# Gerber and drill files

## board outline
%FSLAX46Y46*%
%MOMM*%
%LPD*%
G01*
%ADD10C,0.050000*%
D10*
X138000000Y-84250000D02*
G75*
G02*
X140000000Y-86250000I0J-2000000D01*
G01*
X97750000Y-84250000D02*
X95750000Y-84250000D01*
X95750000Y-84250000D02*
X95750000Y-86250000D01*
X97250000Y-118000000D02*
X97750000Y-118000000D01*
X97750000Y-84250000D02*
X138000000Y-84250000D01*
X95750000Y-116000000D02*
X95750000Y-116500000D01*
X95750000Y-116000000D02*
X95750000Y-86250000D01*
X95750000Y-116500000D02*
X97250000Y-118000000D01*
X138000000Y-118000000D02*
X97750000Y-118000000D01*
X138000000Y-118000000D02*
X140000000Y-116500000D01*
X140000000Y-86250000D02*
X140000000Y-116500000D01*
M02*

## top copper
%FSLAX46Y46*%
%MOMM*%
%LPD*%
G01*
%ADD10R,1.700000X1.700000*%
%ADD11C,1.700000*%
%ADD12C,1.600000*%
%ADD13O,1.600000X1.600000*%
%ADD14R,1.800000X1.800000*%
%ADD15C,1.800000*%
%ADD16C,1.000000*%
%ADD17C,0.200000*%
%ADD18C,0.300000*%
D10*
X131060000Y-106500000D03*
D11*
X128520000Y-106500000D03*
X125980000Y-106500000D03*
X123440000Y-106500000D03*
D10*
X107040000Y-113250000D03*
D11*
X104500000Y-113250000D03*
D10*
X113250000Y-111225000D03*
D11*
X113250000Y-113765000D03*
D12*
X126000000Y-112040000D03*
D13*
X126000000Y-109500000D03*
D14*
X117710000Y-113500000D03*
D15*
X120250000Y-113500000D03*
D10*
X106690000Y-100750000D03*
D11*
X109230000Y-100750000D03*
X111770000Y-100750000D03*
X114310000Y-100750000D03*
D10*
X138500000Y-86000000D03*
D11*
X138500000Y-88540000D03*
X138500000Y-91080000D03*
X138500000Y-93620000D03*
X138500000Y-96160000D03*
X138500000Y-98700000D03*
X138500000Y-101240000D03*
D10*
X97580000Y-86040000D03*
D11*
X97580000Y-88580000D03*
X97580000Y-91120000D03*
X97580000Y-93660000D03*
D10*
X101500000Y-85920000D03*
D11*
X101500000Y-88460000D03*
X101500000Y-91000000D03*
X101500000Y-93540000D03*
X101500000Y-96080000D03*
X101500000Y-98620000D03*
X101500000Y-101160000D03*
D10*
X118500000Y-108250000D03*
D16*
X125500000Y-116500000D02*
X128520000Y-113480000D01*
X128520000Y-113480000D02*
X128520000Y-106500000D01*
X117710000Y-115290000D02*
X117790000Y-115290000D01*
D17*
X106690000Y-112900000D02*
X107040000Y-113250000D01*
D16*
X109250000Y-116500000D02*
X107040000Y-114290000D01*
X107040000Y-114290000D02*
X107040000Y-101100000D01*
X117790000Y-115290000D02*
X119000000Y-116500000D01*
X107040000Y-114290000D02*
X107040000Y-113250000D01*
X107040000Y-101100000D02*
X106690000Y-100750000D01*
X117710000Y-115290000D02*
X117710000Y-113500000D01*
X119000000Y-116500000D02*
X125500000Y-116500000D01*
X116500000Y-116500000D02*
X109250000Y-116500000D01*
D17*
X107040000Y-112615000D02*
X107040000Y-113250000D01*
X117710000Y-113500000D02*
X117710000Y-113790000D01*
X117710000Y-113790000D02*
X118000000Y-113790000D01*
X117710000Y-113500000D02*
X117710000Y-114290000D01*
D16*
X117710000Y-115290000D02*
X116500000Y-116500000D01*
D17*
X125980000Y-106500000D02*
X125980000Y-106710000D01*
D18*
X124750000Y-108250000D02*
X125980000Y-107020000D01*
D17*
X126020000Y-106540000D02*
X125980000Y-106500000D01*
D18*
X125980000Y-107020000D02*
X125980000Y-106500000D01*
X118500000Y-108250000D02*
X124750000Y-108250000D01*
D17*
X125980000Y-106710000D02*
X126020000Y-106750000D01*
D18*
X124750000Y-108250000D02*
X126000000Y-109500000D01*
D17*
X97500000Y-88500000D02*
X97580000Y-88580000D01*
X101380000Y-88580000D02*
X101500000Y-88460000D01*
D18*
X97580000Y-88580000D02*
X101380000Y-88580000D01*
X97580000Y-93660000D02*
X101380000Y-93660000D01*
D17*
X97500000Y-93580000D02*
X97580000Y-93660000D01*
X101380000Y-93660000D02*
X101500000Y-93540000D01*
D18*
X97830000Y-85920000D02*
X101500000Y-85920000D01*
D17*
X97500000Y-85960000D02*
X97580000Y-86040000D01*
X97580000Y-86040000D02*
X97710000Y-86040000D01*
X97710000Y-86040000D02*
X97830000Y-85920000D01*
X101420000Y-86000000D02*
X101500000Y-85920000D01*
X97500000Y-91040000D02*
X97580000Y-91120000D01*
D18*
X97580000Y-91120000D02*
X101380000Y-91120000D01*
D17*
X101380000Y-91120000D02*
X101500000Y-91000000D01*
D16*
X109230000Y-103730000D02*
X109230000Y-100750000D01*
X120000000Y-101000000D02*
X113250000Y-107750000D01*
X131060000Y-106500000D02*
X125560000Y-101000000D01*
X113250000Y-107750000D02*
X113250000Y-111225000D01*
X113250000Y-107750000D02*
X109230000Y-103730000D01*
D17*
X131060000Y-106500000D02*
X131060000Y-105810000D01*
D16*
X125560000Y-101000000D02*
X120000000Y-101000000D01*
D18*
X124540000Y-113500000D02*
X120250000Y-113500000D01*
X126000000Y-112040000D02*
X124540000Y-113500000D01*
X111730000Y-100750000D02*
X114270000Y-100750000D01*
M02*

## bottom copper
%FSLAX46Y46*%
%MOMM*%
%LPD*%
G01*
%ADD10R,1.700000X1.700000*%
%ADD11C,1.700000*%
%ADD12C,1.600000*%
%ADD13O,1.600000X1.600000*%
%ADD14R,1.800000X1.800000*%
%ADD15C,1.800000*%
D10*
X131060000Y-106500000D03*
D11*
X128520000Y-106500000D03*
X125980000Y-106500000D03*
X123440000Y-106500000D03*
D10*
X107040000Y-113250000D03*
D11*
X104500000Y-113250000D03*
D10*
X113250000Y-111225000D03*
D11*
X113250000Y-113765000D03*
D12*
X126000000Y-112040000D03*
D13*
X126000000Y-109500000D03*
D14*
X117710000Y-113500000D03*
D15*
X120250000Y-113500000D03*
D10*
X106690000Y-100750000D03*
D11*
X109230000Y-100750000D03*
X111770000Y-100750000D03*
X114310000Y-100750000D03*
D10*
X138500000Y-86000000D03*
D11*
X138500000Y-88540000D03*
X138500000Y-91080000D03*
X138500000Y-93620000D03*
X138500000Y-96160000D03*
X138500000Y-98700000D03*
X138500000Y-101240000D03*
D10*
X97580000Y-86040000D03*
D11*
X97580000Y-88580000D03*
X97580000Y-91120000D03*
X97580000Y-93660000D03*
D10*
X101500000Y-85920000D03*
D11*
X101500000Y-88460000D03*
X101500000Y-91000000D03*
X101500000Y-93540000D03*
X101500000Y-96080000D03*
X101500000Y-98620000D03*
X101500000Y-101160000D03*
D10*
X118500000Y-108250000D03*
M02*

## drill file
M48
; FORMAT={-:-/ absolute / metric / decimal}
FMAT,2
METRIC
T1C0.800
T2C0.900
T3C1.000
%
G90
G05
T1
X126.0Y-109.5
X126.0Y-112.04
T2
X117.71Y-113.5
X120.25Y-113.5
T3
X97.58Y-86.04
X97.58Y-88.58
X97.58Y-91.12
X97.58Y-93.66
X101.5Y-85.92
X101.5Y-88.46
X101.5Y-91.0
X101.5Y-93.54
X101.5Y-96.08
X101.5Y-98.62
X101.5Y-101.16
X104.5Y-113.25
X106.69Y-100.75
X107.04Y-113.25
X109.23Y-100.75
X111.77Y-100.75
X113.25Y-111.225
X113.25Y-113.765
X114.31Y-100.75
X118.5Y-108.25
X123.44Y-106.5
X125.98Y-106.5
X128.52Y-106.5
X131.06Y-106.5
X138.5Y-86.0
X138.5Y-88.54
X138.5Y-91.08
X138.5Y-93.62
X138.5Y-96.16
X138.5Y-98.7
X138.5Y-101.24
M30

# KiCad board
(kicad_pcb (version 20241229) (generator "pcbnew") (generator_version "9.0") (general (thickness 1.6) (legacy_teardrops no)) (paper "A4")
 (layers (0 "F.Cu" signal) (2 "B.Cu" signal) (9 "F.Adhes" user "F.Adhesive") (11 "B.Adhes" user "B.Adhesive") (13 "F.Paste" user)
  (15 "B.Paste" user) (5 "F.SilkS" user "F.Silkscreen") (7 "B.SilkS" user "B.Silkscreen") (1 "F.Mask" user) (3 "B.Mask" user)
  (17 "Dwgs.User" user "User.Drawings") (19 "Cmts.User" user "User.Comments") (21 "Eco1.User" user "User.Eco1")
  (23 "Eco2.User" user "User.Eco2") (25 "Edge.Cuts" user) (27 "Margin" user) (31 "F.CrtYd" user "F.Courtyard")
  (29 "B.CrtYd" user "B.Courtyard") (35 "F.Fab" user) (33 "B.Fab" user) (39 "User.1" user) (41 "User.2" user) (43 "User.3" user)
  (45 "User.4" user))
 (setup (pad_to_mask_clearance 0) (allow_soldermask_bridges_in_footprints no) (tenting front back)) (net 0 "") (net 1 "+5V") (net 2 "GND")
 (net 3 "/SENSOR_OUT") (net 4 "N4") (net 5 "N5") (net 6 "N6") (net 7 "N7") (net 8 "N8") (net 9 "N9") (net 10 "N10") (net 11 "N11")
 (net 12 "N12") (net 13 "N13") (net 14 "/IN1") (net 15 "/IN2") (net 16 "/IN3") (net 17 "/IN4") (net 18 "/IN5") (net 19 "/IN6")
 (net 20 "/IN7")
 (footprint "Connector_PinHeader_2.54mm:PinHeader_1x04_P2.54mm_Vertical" (layer "F.Cu") (at 131.06 106.5 -90)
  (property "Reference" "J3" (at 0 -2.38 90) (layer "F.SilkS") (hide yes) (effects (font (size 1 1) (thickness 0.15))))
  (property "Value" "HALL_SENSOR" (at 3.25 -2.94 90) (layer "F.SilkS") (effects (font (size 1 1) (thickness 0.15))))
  (pad "1" thru_hole rect (at 0 0 270) (size 1.7 1.7) (drill 1) (layers "*.Cu" "*.Mask") (remove_unused_layers no) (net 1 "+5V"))
  (pad "2" thru_hole circle (at 0 2.54 270) (size 1.7 1.7) (drill 1) (layers "*.Cu" "*.Mask") (remove_unused_layers no) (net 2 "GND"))
  (pad "3" thru_hole circle (at 0 5.08 270) (size 1.7 1.7) (drill 1) (layers "*.Cu" "*.Mask") (remove_unused_layers no)
   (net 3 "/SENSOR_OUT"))
  (pad "4" thru_hole circle (at 0 7.62 270) (size 1.7 1.7) (drill 1) (layers "*.Cu" "*.Mask") (remove_unused_layers no) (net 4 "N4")))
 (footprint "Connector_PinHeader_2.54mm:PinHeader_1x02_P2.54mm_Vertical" (layer "F.Cu") (at 107.04 113.25 -90)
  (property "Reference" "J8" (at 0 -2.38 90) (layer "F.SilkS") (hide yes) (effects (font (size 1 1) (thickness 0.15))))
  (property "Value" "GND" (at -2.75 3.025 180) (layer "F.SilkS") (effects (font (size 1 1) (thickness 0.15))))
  (pad "1" thru_hole rect (at 0 0 270) (size 1.7 1.7) (drill 1) (layers "*.Cu" "*.Mask") (remove_unused_layers no) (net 2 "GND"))
  (pad "2" thru_hole circle (at 0 2.54 270) (size 1.7 1.7) (drill 1) (layers "*.Cu" "*.Mask") (remove_unused_layers no)))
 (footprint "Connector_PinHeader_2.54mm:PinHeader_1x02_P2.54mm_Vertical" (layer "F.Cu") (at 113.25 111.225)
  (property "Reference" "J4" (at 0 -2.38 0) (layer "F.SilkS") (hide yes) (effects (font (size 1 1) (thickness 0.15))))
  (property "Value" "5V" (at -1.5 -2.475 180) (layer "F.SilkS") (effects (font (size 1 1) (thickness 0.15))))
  (pad "1" thru_hole rect (at 0 0) (size 1.7 1.7) (drill 1) (layers "*.Cu" "*.Mask") (remove_unused_layers no) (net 1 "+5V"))
  (pad "2" thru_hole circle (at 0 2.54) (size 1.7 1.7) (drill 1) (layers "*.Cu" "*.Mask") (remove_unused_layers no)))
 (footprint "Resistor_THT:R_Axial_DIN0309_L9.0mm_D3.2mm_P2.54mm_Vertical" (layer "F.Cu") (at 126 112.04 90)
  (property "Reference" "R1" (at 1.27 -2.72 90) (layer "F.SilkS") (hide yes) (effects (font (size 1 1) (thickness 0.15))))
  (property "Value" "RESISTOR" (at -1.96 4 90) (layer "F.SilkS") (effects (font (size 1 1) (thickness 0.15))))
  (pad "1" thru_hole circle (at 0 0 90) (size 1.6 1.6) (drill 0.8) (layers "*.Cu" "*.Mask") (remove_unused_layers no) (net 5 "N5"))
  (pad "2" thru_hole oval (at 2.54 0 90) (size 1.6 1.6) (drill 0.8) (layers "*.Cu" "*.Mask") (remove_unused_layers no) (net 3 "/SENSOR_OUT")))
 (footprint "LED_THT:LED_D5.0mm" (layer "F.Cu") (at 117.71 113.5)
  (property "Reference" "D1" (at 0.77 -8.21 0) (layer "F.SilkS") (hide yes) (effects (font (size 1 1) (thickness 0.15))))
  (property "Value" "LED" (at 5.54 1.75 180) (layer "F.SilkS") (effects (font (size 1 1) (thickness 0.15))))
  (pad "1" thru_hole rect (at 0 0) (size 1.8 1.8) (drill 0.9) (layers "*.Cu" "*.Mask") (remove_unused_layers no) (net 2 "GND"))
  (pad "2" thru_hole circle (at 2.54 0) (size 1.8 1.8) (drill 0.9) (layers "*.Cu" "*.Mask") (remove_unused_layers no) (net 5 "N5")))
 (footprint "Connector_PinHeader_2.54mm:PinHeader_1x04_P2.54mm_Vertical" (layer "F.Cu") (at 106.69 100.75 90)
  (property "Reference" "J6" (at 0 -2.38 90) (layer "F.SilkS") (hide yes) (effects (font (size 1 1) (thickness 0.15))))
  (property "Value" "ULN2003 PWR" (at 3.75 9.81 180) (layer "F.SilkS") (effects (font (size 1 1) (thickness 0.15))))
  (pad "1" thru_hole rect (at 0 0 90) (size 1.7 1.7) (drill 1) (layers "*.Cu" "*.Mask") (remove_unused_layers no) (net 2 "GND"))
  (pad "2" thru_hole circle (at 0 2.54 90) (size 1.7 1.7) (drill 1) (layers "*.Cu" "*.Mask") (remove_unused_layers no) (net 1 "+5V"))
  (pad "3" thru_hole circle (at 0 5.08 90) (size 1.7 1.7) (drill 1) (layers "*.Cu" "*.Mask") (remove_unused_layers no) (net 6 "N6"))
  (pad "4" thru_hole circle (at 0 7.62 90) (size 1.7 1.7) (drill 1) (layers "*.Cu" "*.Mask") (remove_unused_layers no) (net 6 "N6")))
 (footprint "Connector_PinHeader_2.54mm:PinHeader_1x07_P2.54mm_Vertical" (layer "F.Cu") (at 138.5 86)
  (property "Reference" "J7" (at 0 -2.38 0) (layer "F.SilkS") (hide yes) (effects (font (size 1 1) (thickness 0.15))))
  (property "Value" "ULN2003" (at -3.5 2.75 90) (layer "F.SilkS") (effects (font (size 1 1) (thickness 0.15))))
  (pad "1" thru_hole rect (at 0 0) (size 1.7 1.7) (drill 1) (layers "*.Cu" "*.Mask") (remove_unused_layers no) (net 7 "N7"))
  (pad "2" thru_hole circle (at 0 2.54) (size 1.7 1.7) (drill 1) (layers "*.Cu" "*.Mask") (remove_unused_layers no) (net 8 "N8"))
  (pad "3" thru_hole circle (at 0 5.08) (size 1.7 1.7) (drill 1) (layers "*.Cu" "*.Mask") (remove_unused_layers no) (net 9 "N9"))
  (pad "4" thru_hole circle (at 0 7.62) (size 1.7 1.7) (drill 1) (layers "*.Cu" "*.Mask") (remove_unused_layers no) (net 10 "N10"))
  (pad "5" thru_hole circle (at 0 10.16) (size 1.7 1.7) (drill 1) (layers "*.Cu" "*.Mask") (remove_unused_layers no) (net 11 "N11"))
  (pad "6" thru_hole circle (at 0 12.7) (size 1.7 1.7) (drill 1) (layers "*.Cu" "*.Mask") (remove_unused_layers no) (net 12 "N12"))
  (pad "7" thru_hole circle (at 0 15.24) (size 1.7 1.7) (drill 1) (layers "*.Cu" "*.Mask") (remove_unused_layers no) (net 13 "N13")))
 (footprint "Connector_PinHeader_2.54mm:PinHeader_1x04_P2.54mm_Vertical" (layer "F.Cu") (at 97.58 86.04)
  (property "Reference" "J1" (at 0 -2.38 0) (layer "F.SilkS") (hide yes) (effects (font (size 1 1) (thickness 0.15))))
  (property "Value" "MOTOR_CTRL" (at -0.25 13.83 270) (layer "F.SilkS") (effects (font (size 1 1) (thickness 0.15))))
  (pad "1" thru_hole rect (at 0 0) (size 1.7 1.7) (drill 1) (layers "*.Cu" "*.Mask") (remove_unused_layers no) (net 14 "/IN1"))
  (pad "2" thru_hole circle (at 0 2.54) (size 1.7 1.7) (drill 1) (layers "*.Cu" "*.Mask") (remove_unused_layers no) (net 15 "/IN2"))
  (pad "3" thru_hole circle (at 0 5.08) (size 1.7 1.7) (drill 1) (layers "*.Cu" "*.Mask") (remove_unused_layers no) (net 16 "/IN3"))
  (pad "4" thru_hole circle (at 0 7.62) (size 1.7 1.7) (drill 1) (layers "*.Cu" "*.Mask") (remove_unused_layers no) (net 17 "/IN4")))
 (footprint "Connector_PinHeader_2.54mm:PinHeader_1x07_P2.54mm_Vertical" (layer "F.Cu") (at 101.5 85.92)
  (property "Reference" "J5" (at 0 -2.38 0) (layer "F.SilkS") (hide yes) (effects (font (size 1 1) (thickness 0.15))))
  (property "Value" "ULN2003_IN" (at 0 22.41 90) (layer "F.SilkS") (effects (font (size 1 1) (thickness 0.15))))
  (pad "1" thru_hole rect (at 0 0) (size 1.7 1.7) (drill 1) (layers "*.Cu" "*.Mask") (remove_unused_layers no) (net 14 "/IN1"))
  (pad "2" thru_hole circle (at 0 2.54) (size 1.7 1.7) (drill 1) (layers "*.Cu" "*.Mask") (remove_unused_layers no) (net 15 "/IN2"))
  (pad "3" thru_hole circle (at 0 5.08) (size 1.7 1.7) (drill 1) (layers "*.Cu" "*.Mask") (remove_unused_layers no) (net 16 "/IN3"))
  (pad "4" thru_hole circle (at 0 7.62) (size 1.7 1.7) (drill 1) (layers "*.Cu" "*.Mask") (remove_unused_layers no) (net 17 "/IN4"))
  (pad "5" thru_hole circle (at 0 10.16) (size 1.7 1.7) (drill 1) (layers "*.Cu" "*.Mask") (remove_unused_layers no) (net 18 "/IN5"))
  (pad "6" thru_hole circle (at 0 12.7) (size 1.7 1.7) (drill 1) (layers "*.Cu" "*.Mask") (remove_unused_layers no) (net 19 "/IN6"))
  (pad "7" thru_hole circle (at 0 15.24) (size 1.7 1.7) (drill 1) (layers "*.Cu" "*.Mask") (remove_unused_layers no) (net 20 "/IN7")))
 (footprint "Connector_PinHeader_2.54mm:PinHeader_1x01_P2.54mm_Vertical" (layer "F.Cu") (at 118.5 108.25)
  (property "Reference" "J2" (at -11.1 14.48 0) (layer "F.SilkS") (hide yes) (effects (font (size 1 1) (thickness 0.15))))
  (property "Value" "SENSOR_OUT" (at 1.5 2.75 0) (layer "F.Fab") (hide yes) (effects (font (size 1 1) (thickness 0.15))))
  (pad "1" thru_hole rect (at 0 0) (size 1.7 1.7) (drill 1) (layers "*.Cu" "*.Mask") (remove_unused_layers no) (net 3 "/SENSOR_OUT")))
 (gr_arc (start 138 84.25) (mid 139.414214 84.835786) (end 140 86.25) (stroke (width 0.05) (type default)) (layer "Edge.Cuts"))
 (gr_line (start 97.75 84.25) (end 95.75 84.25) (stroke (width 0.05) (type default)) (layer "Edge.Cuts"))
 (gr_line (start 95.75 84.25) (end 95.75 86.25) (stroke (width 0.05) (type default)) (layer "Edge.Cuts"))
 (gr_line (start 97.25 118) (end 97.75 118) (stroke (width 0.05) (type default)) (layer "Edge.Cuts"))
 (gr_line (start 97.75 84.25) (end 138 84.25) (stroke (width 0.05) (type default)) (layer "Edge.Cuts"))
 (gr_line (start 95.75 116) (end 95.75 116.5) (stroke (width 0.05) (type default)) (layer "Edge.Cuts"))
 (gr_line (start 95.75 116) (end 95.75 86.25) (stroke (width 0.05) (type default)) (layer "Edge.Cuts"))
 (gr_line (start 95.75 116.5) (end 97.25 118) (stroke (width 0.05) (type default)) (layer "Edge.Cuts"))
 (gr_line (start 138 118) (end 97.75 118) (stroke (width 0.05) (type default)) (layer "Edge.Cuts"))
 (gr_line (start 138 118) (end 140 116.5) (stroke (width 0.05) (type default)) (layer "Edge.Cuts"))
 (gr_line (start 140 86.25) (end 140 116.5) (stroke (width 0.05) (type default)) (layer "Edge.Cuts"))
 (segment (start 125.5 116.5) (end 128.52 113.48) (width 1) (layer "F.Cu") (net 2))
 (segment (start 128.52 113.48) (end 128.52 106.5) (width 1) (layer "F.Cu") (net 2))
 (segment (start 117.71 115.29) (end 117.79 115.29) (width 1) (layer "F.Cu") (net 2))
 (segment (start 106.69 112.9) (end 107.04 113.25) (width 0.2) (layer "F.Cu") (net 2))
 (segment (start 109.25 116.5) (end 107.04 114.29) (width 1) (layer "F.Cu") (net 2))
 (segment (start 107.04 114.29) (end 107.04 101.1) (width 1) (layer "F.Cu") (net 2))
 (segment (start 117.79 115.29) (end 119 116.5) (width 1) (layer "F.Cu") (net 2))
 (segment (start 107.04 114.29) (end 107.04 113.25) (width 1) (layer "F.Cu") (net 2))
 (segment (start 107.04 101.1) (end 106.69 100.75) (width 1) (layer "F.Cu") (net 2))
 (segment (start 117.71 115.29) (end 117.71 113.5) (width 1) (layer "F.Cu") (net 2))
 (segment (start 119 116.5) (end 125.5 116.5) (width 1) (layer "F.Cu") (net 2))
 (segment (start 116.5 116.5) (end 109.25 116.5) (width 1) (layer "F.Cu") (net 2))
 (segment (start 107.04 112.615) (end 107.04 113.25) (width 0.2) (layer "F.Cu") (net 2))
 (segment (start 117.71 113.5) (end 117.71 113.79) (width 0.2) (layer "F.Cu") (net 2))
 (segment (start 117.71 113.79) (end 118 113.79) (width 0.2) (layer "F.Cu") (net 2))
 (segment (start 117.71 113.5) (end 117.71 114.29) (width 0.2) (layer "F.Cu") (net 2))
 (segment (start 117.71 115.29) (end 116.5 116.5) (width 1) (layer "F.Cu") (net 2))
 (segment (start 125.98 106.5) (end 125.98 106.71) (width 0.2) (layer "F.Cu") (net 3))
 (segment (start 124.75 108.25) (end 125.98 107.02) (width 0.3) (layer "F.Cu") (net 3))
 (segment (start 126.02 106.54) (end 125.98 106.5) (width 0.2) (layer "F.Cu") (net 3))
 (segment (start 125.98 107.02) (end 125.98 106.5) (width 0.3) (layer "F.Cu") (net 3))
 (segment (start 118.5 108.25) (end 124.75 108.25) (width 0.3) (layer "F.Cu") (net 3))
 (segment (start 125.98 106.71) (end 126.02 106.75) (width 0.2) (layer "F.Cu") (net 3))
 (segment (start 124.75 108.25) (end 126 109.5) (width 0.3) (layer "F.Cu") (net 3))
 (segment (start 97.5 88.5) (end 97.58 88.58) (width 0.2) (layer "F.Cu") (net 15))
 (segment (start 101.38 88.58) (end 101.5 88.46) (width 0.2) (layer "F.Cu") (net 15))
 (segment (start 97.58 88.58) (end 101.38 88.58) (width 0.3) (layer "F.Cu") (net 15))
 (segment (start 97.58 93.66) (end 101.38 93.66) (width 0.3) (layer "F.Cu") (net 17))
 (segment (start 97.5 93.58) (end 97.58 93.66) (width 0.2) (layer "F.Cu") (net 17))
 (segment (start 101.38 93.66) (end 101.5 93.54) (width 0.2) (layer "F.Cu") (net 17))
 (segment (start 97.83 85.92) (end 101.5 85.92) (width 0.3) (layer "F.Cu") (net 14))
 (segment (start 97.5 85.96) (end 97.58 86.04) (width 0.2) (layer "F.Cu") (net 14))
 (segment (start 97.58 86.04) (end 97.71 86.04) (width 0.2) (layer "F.Cu") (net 14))
 (segment (start 97.71 86.04) (end 97.83 85.92) (width 0.2) (layer "F.Cu") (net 14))
 (segment (start 101.42 86) (end 101.5 85.92) (width 0.2) (layer "F.Cu") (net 14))
 (segment (start 97.5 91.04) (end 97.58 91.12) (width 0.2) (layer "F.Cu") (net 16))
 (segment (start 97.58 91.12) (end 101.38 91.12) (width 0.3) (layer "F.Cu") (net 16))
 (segment (start 101.38 91.12) (end 101.5 91) (width 0.2) (layer "F.Cu") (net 16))
 (segment (start 109.23 103.73) (end 109.23 100.75) (width 1) (layer "F.Cu") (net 1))
 (segment (start 120 101) (end 113.25 107.75) (width 1) (layer "F.Cu") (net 1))
 (segment (start 131.06 106.5) (end 125.56 101) (width 1) (layer "F.Cu") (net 1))
 (segment (start 113.25 107.75) (end 113.25 111.225) (width 1) (layer "F.Cu") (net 1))
 (segment (start 113.25 107.75) (end 109.23 103.73) (width 1) (layer "F.Cu") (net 1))
 (segment (start 131.06 106.5) (end 131.06 105.81) (width 0.2) (layer "F.Cu") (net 1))
 (segment (start 125.56 101) (end 120 101) (width 1) (layer "F.Cu") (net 1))
 (segment (start 124.54 113.5) (end 120.25 113.5) (width 0.3) (layer "F.Cu") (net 5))
 (segment (start 126 112.04) (end 124.54 113.5) (width 0.3) (layer "F.Cu") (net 5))
 (segment (start 111.73 100.75) (end 114.27 100.75) (width 0.3) (layer "F.Cu") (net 6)))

